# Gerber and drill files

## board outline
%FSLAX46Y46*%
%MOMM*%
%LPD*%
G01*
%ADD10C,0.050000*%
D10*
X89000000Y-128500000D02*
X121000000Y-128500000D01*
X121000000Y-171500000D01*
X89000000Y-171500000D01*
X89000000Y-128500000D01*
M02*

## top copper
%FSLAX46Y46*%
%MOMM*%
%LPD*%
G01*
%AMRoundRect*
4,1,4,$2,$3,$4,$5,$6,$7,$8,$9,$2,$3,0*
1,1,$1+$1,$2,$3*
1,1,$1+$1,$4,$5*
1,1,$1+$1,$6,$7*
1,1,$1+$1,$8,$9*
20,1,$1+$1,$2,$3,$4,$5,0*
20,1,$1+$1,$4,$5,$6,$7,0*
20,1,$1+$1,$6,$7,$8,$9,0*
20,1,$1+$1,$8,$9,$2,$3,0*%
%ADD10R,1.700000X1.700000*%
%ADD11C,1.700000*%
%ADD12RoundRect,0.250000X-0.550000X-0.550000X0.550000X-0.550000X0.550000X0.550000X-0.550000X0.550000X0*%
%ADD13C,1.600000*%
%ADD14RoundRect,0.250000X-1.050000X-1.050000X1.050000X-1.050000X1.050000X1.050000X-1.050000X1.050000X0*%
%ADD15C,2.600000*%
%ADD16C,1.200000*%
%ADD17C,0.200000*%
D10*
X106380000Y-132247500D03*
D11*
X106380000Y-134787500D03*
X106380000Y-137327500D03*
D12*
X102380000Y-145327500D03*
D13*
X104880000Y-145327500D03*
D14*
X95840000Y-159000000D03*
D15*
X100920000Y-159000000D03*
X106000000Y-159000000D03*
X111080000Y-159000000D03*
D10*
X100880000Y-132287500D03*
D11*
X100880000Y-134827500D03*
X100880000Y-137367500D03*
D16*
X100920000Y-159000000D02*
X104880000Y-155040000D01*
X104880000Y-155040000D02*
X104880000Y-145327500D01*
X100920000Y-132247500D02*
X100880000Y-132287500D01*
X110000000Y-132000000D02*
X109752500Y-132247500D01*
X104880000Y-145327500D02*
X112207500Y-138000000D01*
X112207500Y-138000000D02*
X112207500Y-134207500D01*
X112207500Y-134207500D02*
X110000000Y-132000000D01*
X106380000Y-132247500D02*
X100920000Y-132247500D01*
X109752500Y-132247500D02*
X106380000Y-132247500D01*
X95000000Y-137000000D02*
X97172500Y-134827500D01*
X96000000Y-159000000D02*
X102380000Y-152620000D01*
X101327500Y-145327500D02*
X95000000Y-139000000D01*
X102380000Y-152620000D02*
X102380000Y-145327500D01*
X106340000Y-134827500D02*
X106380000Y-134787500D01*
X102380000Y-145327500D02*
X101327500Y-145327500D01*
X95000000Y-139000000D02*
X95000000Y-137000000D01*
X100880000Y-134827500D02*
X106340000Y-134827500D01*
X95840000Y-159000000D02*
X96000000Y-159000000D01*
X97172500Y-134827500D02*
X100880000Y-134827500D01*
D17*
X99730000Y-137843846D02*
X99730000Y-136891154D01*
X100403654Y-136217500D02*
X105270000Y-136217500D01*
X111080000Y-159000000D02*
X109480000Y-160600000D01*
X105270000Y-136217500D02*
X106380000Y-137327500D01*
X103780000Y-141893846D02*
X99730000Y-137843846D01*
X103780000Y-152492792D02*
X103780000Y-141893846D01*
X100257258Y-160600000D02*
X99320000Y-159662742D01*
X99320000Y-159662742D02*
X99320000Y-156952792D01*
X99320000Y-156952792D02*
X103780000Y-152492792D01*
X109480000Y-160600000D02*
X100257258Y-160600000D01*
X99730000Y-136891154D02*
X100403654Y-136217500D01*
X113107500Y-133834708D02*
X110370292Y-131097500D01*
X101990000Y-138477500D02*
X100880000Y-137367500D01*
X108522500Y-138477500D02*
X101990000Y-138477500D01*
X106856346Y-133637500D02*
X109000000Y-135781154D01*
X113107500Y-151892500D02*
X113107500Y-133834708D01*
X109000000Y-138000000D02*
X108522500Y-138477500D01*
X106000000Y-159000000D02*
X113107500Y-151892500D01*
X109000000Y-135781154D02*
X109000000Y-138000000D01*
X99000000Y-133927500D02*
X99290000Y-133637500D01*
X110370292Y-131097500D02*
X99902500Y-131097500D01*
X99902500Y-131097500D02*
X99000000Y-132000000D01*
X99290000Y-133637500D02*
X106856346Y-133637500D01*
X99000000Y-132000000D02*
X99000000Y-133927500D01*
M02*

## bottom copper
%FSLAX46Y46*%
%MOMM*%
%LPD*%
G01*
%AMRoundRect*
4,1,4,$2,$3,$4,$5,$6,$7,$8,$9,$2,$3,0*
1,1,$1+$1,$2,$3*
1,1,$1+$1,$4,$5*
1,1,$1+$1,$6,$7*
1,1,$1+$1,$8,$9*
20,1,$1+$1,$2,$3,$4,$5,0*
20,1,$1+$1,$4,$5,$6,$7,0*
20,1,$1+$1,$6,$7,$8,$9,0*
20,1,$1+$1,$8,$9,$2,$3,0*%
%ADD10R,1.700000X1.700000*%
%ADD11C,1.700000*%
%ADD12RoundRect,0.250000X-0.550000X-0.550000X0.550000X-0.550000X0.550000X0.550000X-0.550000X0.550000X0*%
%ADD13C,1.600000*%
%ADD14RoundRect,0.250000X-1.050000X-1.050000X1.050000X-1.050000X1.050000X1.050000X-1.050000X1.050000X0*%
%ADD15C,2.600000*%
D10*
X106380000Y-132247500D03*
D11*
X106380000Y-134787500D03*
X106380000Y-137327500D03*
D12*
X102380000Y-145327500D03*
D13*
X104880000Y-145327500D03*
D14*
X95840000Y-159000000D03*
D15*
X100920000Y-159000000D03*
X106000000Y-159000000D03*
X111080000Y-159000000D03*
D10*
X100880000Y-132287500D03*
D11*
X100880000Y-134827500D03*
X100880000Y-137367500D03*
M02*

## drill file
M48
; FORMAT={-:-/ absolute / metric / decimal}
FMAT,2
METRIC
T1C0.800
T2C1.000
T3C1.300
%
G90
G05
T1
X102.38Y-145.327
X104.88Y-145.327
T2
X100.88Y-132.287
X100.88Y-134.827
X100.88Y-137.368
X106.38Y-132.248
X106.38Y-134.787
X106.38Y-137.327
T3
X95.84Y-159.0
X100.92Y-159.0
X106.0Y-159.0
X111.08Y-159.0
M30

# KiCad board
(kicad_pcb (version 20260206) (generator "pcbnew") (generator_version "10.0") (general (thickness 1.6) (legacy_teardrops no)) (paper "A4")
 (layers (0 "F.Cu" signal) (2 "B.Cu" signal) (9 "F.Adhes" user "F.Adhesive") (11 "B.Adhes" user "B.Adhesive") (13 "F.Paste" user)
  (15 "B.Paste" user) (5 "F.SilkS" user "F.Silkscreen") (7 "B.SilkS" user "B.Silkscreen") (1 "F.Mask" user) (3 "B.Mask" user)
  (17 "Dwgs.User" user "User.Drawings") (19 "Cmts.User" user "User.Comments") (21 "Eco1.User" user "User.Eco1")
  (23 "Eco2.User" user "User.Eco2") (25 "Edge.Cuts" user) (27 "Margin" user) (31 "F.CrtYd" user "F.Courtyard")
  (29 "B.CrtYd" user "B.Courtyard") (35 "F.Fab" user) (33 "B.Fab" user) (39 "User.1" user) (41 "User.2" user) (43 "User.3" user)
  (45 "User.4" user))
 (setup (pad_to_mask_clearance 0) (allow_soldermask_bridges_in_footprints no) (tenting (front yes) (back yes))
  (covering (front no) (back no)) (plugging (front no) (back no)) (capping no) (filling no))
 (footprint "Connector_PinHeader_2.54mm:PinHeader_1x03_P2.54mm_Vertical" (layer "F.Cu") (at 106.38 132.2475)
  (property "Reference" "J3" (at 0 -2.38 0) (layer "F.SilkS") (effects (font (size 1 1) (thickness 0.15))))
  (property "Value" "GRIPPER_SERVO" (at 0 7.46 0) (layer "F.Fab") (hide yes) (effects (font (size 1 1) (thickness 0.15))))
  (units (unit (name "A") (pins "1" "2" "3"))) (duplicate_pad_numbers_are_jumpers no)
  (pad "1" thru_hole rect (at 0 0) (size 1.7 1.7) (drill 1) (layers "*.Cu" "*.Mask") (remove_unused_layers no) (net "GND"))
  (pad "2" thru_hole circle (at 0 2.54) (size 1.7 1.7) (drill 1) (layers "*.Cu" "*.Mask") (remove_unused_layers no) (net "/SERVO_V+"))
  (pad "3" thru_hole circle (at 0 5.08) (size 1.7 1.7) (drill 1) (layers "*.Cu" "*.Mask") (remove_unused_layers no) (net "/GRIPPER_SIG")))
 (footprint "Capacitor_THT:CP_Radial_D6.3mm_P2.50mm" (layer "F.Cu") (at 102.38 145.3275)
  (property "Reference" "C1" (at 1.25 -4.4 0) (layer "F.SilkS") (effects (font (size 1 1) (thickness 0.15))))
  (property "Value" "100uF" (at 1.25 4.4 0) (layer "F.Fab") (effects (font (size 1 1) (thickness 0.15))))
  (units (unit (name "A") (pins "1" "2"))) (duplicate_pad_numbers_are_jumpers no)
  (pad "1" thru_hole roundrect (at 0 0) (size 1.6 1.6) (drill 0.8) (layers "*.Cu" "*.Mask") (remove_unused_layers no)
   (roundrect_rratio 0.15625) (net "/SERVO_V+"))
  (pad "2" thru_hole circle (at 2.5 0) (size 1.6 1.6) (drill 0.8) (layers "*.Cu" "*.Mask") (remove_unused_layers no) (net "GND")))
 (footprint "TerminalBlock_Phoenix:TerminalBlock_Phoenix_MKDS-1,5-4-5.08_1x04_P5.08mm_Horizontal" (layer "F.Cu") (at 95.84 159)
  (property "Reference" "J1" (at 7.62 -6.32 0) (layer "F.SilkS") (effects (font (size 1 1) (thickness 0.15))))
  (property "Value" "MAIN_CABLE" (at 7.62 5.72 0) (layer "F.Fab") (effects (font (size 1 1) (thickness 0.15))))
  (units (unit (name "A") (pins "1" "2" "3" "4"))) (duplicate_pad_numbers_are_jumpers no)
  (pad "1" thru_hole roundrect (at 0 0) (size 2.6 2.6) (drill 1.3) (layers "*.Cu" "*.Mask") (remove_unused_layers no)
   (roundrect_rratio 0.096154) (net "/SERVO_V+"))
  (pad "2" thru_hole circle (at 5.08 0) (size 2.6 2.6) (drill 1.3) (layers "*.Cu" "*.Mask") (remove_unused_layers no) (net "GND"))
  (pad "3" thru_hole circle (at 10.16 0) (size 2.6 2.6) (drill 1.3) (layers "*.Cu" "*.Mask") (remove_unused_layers no) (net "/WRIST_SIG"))
  (pad "4" thru_hole circle (at 15.24 0) (size 2.6 2.6) (drill 1.3) (layers "*.Cu" "*.Mask") (remove_unused_layers no) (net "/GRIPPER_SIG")))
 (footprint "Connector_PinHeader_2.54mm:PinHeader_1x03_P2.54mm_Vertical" (layer "F.Cu") (at 100.88 132.2875)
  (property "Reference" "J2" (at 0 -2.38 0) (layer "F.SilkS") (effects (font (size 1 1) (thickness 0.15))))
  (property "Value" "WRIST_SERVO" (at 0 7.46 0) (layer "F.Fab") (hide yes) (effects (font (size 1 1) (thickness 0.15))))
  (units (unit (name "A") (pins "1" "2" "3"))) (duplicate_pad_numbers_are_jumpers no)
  (pad "1" thru_hole rect (at 0 0) (size 1.7 1.7) (drill 1) (layers "*.Cu" "*.Mask") (remove_unused_layers no) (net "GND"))
  (pad "2" thru_hole circle (at 0 2.54) (size 1.7 1.7) (drill 1) (layers "*.Cu" "*.Mask") (remove_unused_layers no) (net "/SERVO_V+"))
  (pad "3" thru_hole circle (at 0 5.08) (size 1.7 1.7) (drill 1) (layers "*.Cu" "*.Mask") (remove_unused_layers no) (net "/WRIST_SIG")))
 (gr_rect (start 89 128.5) (end 121 171.5) (stroke (width 0.05) (type default)) (fill no) (layer "Edge.Cuts"))
 (segment (start 100.92 159) (end 104.88 155.04) (width 1.2) (layer "F.Cu") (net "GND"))
 (segment (start 104.88 155.04) (end 104.88 145.3275) (width 1.2) (layer "F.Cu") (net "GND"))
 (segment (start 100.92 132.2475) (end 100.88 132.2875) (width 1.2) (layer "F.Cu") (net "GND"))
 (segment (start 110 132) (end 109.7525 132.2475) (width 1.2) (layer "F.Cu") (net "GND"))
 (segment (start 104.88 145.3275) (end 112.2075 138) (width 1.2) (layer "F.Cu") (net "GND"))
 (segment (start 112.2075 138) (end 112.2075 134.2075) (width 1.2) (layer "F.Cu") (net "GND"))
 (segment (start 112.2075 134.2075) (end 110 132) (width 1.2) (layer "F.Cu") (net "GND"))
 (segment (start 106.38 132.2475) (end 100.92 132.2475) (width 1.2) (layer "F.Cu") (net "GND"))
 (segment (start 109.7525 132.2475) (end 106.38 132.2475) (width 1.2) (layer "F.Cu") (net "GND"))
 (segment (start 95 137) (end 97.1725 134.8275) (width 1.2) (layer "F.Cu") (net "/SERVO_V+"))
 (segment (start 96 159) (end 102.38 152.62) (width 1.2) (layer "F.Cu") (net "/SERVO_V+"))
 (segment (start 101.3275 145.3275) (end 95 139) (width 1.2) (layer "F.Cu") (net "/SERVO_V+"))
 (segment (start 102.38 152.62) (end 102.38 145.3275) (width 1.2) (layer "F.Cu") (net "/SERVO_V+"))
 (segment (start 106.34 134.8275) (end 106.38 134.7875) (width 1.2) (layer "F.Cu") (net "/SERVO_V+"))
 (segment (start 102.38 145.3275) (end 101.3275 145.3275) (width 1.2) (layer "F.Cu") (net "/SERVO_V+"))
 (segment (start 95 139) (end 95 137) (width 1.2) (layer "F.Cu") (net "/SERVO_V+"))
 (segment (start 100.88 134.8275) (end 106.34 134.8275) (width 1.2) (layer "F.Cu") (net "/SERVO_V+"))
 (segment (start 95.84 159) (end 96 159) (width 1.2) (layer "F.Cu") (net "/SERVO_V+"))
 (segment (start 97.1725 134.8275) (end 100.88 134.8275) (width 1.2) (layer "F.Cu") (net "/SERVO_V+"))
 (segment (start 99.73 137.843846) (end 99.73 136.891154) (width 0.2) (layer "F.Cu") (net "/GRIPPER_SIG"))
 (segment (start 100.403654 136.2175) (end 105.27 136.2175) (width 0.2) (layer "F.Cu") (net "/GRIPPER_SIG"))
 (segment (start 111.08 159) (end 109.48 160.6) (width 0.2) (layer "F.Cu") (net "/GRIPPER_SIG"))
 (segment (start 105.27 136.2175) (end 106.38 137.3275) (width 0.2) (layer "F.Cu") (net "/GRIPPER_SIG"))
 (segment (start 103.78 141.893846) (end 99.73 137.843846) (width 0.2) (layer "F.Cu") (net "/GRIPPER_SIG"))
 (segment (start 103.78 152.492792) (end 103.78 141.893846) (width 0.2) (layer "F.Cu") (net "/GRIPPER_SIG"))
 (segment (start 100.257258 160.6) (end 99.32 159.662742) (width 0.2) (layer "F.Cu") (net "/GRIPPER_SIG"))
 (segment (start 99.32 159.662742) (end 99.32 156.952792) (width 0.2) (layer "F.Cu") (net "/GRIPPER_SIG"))
 (segment (start 99.32 156.952792) (end 103.78 152.492792) (width 0.2) (layer "F.Cu") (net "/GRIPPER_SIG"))
 (segment (start 109.48 160.6) (end 100.257258 160.6) (width 0.2) (layer "F.Cu") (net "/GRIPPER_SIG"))
 (segment (start 99.73 136.891154) (end 100.403654 136.2175) (width 0.2) (layer "F.Cu") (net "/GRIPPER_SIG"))
 (segment (start 113.1075 133.834708) (end 110.370292 131.0975) (width 0.2) (layer "F.Cu") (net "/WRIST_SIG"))
 (segment (start 101.99 138.4775) (end 100.88 137.3675) (width 0.2) (layer "F.Cu") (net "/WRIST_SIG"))
 (segment (start 108.5225 138.4775) (end 101.99 138.4775) (width 0.2) (layer "F.Cu") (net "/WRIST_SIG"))
 (segment (start 106.856346 133.6375) (end 109 135.781154) (width 0.2) (layer "F.Cu") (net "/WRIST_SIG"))
 (segment (start 113.1075 151.8925) (end 113.1075 133.834708) (width 0.2) (layer "F.Cu") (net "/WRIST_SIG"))
 (segment (start 109 138) (end 108.5225 138.4775) (width 0.2) (layer "F.Cu") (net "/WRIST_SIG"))
 (segment (start 106 159) (end 113.1075 151.8925) (width 0.2) (layer "F.Cu") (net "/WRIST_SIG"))
 (segment (start 109 135.781154) (end 109 138) (width 0.2) (layer "F.Cu") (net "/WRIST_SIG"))
 (segment (start 99 133.9275) (end 99.29 133.6375) (width 0.2) (layer "F.Cu") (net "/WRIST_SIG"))
 (segment (start 110.370292 131.0975) (end 99.9025 131.0975) (width 0.2) (layer "F.Cu") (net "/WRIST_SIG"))
 (segment (start 99.9025 131.0975) (end 99 132) (width 0.2) (layer "F.Cu") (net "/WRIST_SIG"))
 (segment (start 99.29 133.6375) (end 106.856346 133.6375) (width 0.2) (layer "F.Cu") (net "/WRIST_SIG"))
 (segment (start 99 132) (end 99 133.9275) (width 0.2) (layer "F.Cu") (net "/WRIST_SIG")))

